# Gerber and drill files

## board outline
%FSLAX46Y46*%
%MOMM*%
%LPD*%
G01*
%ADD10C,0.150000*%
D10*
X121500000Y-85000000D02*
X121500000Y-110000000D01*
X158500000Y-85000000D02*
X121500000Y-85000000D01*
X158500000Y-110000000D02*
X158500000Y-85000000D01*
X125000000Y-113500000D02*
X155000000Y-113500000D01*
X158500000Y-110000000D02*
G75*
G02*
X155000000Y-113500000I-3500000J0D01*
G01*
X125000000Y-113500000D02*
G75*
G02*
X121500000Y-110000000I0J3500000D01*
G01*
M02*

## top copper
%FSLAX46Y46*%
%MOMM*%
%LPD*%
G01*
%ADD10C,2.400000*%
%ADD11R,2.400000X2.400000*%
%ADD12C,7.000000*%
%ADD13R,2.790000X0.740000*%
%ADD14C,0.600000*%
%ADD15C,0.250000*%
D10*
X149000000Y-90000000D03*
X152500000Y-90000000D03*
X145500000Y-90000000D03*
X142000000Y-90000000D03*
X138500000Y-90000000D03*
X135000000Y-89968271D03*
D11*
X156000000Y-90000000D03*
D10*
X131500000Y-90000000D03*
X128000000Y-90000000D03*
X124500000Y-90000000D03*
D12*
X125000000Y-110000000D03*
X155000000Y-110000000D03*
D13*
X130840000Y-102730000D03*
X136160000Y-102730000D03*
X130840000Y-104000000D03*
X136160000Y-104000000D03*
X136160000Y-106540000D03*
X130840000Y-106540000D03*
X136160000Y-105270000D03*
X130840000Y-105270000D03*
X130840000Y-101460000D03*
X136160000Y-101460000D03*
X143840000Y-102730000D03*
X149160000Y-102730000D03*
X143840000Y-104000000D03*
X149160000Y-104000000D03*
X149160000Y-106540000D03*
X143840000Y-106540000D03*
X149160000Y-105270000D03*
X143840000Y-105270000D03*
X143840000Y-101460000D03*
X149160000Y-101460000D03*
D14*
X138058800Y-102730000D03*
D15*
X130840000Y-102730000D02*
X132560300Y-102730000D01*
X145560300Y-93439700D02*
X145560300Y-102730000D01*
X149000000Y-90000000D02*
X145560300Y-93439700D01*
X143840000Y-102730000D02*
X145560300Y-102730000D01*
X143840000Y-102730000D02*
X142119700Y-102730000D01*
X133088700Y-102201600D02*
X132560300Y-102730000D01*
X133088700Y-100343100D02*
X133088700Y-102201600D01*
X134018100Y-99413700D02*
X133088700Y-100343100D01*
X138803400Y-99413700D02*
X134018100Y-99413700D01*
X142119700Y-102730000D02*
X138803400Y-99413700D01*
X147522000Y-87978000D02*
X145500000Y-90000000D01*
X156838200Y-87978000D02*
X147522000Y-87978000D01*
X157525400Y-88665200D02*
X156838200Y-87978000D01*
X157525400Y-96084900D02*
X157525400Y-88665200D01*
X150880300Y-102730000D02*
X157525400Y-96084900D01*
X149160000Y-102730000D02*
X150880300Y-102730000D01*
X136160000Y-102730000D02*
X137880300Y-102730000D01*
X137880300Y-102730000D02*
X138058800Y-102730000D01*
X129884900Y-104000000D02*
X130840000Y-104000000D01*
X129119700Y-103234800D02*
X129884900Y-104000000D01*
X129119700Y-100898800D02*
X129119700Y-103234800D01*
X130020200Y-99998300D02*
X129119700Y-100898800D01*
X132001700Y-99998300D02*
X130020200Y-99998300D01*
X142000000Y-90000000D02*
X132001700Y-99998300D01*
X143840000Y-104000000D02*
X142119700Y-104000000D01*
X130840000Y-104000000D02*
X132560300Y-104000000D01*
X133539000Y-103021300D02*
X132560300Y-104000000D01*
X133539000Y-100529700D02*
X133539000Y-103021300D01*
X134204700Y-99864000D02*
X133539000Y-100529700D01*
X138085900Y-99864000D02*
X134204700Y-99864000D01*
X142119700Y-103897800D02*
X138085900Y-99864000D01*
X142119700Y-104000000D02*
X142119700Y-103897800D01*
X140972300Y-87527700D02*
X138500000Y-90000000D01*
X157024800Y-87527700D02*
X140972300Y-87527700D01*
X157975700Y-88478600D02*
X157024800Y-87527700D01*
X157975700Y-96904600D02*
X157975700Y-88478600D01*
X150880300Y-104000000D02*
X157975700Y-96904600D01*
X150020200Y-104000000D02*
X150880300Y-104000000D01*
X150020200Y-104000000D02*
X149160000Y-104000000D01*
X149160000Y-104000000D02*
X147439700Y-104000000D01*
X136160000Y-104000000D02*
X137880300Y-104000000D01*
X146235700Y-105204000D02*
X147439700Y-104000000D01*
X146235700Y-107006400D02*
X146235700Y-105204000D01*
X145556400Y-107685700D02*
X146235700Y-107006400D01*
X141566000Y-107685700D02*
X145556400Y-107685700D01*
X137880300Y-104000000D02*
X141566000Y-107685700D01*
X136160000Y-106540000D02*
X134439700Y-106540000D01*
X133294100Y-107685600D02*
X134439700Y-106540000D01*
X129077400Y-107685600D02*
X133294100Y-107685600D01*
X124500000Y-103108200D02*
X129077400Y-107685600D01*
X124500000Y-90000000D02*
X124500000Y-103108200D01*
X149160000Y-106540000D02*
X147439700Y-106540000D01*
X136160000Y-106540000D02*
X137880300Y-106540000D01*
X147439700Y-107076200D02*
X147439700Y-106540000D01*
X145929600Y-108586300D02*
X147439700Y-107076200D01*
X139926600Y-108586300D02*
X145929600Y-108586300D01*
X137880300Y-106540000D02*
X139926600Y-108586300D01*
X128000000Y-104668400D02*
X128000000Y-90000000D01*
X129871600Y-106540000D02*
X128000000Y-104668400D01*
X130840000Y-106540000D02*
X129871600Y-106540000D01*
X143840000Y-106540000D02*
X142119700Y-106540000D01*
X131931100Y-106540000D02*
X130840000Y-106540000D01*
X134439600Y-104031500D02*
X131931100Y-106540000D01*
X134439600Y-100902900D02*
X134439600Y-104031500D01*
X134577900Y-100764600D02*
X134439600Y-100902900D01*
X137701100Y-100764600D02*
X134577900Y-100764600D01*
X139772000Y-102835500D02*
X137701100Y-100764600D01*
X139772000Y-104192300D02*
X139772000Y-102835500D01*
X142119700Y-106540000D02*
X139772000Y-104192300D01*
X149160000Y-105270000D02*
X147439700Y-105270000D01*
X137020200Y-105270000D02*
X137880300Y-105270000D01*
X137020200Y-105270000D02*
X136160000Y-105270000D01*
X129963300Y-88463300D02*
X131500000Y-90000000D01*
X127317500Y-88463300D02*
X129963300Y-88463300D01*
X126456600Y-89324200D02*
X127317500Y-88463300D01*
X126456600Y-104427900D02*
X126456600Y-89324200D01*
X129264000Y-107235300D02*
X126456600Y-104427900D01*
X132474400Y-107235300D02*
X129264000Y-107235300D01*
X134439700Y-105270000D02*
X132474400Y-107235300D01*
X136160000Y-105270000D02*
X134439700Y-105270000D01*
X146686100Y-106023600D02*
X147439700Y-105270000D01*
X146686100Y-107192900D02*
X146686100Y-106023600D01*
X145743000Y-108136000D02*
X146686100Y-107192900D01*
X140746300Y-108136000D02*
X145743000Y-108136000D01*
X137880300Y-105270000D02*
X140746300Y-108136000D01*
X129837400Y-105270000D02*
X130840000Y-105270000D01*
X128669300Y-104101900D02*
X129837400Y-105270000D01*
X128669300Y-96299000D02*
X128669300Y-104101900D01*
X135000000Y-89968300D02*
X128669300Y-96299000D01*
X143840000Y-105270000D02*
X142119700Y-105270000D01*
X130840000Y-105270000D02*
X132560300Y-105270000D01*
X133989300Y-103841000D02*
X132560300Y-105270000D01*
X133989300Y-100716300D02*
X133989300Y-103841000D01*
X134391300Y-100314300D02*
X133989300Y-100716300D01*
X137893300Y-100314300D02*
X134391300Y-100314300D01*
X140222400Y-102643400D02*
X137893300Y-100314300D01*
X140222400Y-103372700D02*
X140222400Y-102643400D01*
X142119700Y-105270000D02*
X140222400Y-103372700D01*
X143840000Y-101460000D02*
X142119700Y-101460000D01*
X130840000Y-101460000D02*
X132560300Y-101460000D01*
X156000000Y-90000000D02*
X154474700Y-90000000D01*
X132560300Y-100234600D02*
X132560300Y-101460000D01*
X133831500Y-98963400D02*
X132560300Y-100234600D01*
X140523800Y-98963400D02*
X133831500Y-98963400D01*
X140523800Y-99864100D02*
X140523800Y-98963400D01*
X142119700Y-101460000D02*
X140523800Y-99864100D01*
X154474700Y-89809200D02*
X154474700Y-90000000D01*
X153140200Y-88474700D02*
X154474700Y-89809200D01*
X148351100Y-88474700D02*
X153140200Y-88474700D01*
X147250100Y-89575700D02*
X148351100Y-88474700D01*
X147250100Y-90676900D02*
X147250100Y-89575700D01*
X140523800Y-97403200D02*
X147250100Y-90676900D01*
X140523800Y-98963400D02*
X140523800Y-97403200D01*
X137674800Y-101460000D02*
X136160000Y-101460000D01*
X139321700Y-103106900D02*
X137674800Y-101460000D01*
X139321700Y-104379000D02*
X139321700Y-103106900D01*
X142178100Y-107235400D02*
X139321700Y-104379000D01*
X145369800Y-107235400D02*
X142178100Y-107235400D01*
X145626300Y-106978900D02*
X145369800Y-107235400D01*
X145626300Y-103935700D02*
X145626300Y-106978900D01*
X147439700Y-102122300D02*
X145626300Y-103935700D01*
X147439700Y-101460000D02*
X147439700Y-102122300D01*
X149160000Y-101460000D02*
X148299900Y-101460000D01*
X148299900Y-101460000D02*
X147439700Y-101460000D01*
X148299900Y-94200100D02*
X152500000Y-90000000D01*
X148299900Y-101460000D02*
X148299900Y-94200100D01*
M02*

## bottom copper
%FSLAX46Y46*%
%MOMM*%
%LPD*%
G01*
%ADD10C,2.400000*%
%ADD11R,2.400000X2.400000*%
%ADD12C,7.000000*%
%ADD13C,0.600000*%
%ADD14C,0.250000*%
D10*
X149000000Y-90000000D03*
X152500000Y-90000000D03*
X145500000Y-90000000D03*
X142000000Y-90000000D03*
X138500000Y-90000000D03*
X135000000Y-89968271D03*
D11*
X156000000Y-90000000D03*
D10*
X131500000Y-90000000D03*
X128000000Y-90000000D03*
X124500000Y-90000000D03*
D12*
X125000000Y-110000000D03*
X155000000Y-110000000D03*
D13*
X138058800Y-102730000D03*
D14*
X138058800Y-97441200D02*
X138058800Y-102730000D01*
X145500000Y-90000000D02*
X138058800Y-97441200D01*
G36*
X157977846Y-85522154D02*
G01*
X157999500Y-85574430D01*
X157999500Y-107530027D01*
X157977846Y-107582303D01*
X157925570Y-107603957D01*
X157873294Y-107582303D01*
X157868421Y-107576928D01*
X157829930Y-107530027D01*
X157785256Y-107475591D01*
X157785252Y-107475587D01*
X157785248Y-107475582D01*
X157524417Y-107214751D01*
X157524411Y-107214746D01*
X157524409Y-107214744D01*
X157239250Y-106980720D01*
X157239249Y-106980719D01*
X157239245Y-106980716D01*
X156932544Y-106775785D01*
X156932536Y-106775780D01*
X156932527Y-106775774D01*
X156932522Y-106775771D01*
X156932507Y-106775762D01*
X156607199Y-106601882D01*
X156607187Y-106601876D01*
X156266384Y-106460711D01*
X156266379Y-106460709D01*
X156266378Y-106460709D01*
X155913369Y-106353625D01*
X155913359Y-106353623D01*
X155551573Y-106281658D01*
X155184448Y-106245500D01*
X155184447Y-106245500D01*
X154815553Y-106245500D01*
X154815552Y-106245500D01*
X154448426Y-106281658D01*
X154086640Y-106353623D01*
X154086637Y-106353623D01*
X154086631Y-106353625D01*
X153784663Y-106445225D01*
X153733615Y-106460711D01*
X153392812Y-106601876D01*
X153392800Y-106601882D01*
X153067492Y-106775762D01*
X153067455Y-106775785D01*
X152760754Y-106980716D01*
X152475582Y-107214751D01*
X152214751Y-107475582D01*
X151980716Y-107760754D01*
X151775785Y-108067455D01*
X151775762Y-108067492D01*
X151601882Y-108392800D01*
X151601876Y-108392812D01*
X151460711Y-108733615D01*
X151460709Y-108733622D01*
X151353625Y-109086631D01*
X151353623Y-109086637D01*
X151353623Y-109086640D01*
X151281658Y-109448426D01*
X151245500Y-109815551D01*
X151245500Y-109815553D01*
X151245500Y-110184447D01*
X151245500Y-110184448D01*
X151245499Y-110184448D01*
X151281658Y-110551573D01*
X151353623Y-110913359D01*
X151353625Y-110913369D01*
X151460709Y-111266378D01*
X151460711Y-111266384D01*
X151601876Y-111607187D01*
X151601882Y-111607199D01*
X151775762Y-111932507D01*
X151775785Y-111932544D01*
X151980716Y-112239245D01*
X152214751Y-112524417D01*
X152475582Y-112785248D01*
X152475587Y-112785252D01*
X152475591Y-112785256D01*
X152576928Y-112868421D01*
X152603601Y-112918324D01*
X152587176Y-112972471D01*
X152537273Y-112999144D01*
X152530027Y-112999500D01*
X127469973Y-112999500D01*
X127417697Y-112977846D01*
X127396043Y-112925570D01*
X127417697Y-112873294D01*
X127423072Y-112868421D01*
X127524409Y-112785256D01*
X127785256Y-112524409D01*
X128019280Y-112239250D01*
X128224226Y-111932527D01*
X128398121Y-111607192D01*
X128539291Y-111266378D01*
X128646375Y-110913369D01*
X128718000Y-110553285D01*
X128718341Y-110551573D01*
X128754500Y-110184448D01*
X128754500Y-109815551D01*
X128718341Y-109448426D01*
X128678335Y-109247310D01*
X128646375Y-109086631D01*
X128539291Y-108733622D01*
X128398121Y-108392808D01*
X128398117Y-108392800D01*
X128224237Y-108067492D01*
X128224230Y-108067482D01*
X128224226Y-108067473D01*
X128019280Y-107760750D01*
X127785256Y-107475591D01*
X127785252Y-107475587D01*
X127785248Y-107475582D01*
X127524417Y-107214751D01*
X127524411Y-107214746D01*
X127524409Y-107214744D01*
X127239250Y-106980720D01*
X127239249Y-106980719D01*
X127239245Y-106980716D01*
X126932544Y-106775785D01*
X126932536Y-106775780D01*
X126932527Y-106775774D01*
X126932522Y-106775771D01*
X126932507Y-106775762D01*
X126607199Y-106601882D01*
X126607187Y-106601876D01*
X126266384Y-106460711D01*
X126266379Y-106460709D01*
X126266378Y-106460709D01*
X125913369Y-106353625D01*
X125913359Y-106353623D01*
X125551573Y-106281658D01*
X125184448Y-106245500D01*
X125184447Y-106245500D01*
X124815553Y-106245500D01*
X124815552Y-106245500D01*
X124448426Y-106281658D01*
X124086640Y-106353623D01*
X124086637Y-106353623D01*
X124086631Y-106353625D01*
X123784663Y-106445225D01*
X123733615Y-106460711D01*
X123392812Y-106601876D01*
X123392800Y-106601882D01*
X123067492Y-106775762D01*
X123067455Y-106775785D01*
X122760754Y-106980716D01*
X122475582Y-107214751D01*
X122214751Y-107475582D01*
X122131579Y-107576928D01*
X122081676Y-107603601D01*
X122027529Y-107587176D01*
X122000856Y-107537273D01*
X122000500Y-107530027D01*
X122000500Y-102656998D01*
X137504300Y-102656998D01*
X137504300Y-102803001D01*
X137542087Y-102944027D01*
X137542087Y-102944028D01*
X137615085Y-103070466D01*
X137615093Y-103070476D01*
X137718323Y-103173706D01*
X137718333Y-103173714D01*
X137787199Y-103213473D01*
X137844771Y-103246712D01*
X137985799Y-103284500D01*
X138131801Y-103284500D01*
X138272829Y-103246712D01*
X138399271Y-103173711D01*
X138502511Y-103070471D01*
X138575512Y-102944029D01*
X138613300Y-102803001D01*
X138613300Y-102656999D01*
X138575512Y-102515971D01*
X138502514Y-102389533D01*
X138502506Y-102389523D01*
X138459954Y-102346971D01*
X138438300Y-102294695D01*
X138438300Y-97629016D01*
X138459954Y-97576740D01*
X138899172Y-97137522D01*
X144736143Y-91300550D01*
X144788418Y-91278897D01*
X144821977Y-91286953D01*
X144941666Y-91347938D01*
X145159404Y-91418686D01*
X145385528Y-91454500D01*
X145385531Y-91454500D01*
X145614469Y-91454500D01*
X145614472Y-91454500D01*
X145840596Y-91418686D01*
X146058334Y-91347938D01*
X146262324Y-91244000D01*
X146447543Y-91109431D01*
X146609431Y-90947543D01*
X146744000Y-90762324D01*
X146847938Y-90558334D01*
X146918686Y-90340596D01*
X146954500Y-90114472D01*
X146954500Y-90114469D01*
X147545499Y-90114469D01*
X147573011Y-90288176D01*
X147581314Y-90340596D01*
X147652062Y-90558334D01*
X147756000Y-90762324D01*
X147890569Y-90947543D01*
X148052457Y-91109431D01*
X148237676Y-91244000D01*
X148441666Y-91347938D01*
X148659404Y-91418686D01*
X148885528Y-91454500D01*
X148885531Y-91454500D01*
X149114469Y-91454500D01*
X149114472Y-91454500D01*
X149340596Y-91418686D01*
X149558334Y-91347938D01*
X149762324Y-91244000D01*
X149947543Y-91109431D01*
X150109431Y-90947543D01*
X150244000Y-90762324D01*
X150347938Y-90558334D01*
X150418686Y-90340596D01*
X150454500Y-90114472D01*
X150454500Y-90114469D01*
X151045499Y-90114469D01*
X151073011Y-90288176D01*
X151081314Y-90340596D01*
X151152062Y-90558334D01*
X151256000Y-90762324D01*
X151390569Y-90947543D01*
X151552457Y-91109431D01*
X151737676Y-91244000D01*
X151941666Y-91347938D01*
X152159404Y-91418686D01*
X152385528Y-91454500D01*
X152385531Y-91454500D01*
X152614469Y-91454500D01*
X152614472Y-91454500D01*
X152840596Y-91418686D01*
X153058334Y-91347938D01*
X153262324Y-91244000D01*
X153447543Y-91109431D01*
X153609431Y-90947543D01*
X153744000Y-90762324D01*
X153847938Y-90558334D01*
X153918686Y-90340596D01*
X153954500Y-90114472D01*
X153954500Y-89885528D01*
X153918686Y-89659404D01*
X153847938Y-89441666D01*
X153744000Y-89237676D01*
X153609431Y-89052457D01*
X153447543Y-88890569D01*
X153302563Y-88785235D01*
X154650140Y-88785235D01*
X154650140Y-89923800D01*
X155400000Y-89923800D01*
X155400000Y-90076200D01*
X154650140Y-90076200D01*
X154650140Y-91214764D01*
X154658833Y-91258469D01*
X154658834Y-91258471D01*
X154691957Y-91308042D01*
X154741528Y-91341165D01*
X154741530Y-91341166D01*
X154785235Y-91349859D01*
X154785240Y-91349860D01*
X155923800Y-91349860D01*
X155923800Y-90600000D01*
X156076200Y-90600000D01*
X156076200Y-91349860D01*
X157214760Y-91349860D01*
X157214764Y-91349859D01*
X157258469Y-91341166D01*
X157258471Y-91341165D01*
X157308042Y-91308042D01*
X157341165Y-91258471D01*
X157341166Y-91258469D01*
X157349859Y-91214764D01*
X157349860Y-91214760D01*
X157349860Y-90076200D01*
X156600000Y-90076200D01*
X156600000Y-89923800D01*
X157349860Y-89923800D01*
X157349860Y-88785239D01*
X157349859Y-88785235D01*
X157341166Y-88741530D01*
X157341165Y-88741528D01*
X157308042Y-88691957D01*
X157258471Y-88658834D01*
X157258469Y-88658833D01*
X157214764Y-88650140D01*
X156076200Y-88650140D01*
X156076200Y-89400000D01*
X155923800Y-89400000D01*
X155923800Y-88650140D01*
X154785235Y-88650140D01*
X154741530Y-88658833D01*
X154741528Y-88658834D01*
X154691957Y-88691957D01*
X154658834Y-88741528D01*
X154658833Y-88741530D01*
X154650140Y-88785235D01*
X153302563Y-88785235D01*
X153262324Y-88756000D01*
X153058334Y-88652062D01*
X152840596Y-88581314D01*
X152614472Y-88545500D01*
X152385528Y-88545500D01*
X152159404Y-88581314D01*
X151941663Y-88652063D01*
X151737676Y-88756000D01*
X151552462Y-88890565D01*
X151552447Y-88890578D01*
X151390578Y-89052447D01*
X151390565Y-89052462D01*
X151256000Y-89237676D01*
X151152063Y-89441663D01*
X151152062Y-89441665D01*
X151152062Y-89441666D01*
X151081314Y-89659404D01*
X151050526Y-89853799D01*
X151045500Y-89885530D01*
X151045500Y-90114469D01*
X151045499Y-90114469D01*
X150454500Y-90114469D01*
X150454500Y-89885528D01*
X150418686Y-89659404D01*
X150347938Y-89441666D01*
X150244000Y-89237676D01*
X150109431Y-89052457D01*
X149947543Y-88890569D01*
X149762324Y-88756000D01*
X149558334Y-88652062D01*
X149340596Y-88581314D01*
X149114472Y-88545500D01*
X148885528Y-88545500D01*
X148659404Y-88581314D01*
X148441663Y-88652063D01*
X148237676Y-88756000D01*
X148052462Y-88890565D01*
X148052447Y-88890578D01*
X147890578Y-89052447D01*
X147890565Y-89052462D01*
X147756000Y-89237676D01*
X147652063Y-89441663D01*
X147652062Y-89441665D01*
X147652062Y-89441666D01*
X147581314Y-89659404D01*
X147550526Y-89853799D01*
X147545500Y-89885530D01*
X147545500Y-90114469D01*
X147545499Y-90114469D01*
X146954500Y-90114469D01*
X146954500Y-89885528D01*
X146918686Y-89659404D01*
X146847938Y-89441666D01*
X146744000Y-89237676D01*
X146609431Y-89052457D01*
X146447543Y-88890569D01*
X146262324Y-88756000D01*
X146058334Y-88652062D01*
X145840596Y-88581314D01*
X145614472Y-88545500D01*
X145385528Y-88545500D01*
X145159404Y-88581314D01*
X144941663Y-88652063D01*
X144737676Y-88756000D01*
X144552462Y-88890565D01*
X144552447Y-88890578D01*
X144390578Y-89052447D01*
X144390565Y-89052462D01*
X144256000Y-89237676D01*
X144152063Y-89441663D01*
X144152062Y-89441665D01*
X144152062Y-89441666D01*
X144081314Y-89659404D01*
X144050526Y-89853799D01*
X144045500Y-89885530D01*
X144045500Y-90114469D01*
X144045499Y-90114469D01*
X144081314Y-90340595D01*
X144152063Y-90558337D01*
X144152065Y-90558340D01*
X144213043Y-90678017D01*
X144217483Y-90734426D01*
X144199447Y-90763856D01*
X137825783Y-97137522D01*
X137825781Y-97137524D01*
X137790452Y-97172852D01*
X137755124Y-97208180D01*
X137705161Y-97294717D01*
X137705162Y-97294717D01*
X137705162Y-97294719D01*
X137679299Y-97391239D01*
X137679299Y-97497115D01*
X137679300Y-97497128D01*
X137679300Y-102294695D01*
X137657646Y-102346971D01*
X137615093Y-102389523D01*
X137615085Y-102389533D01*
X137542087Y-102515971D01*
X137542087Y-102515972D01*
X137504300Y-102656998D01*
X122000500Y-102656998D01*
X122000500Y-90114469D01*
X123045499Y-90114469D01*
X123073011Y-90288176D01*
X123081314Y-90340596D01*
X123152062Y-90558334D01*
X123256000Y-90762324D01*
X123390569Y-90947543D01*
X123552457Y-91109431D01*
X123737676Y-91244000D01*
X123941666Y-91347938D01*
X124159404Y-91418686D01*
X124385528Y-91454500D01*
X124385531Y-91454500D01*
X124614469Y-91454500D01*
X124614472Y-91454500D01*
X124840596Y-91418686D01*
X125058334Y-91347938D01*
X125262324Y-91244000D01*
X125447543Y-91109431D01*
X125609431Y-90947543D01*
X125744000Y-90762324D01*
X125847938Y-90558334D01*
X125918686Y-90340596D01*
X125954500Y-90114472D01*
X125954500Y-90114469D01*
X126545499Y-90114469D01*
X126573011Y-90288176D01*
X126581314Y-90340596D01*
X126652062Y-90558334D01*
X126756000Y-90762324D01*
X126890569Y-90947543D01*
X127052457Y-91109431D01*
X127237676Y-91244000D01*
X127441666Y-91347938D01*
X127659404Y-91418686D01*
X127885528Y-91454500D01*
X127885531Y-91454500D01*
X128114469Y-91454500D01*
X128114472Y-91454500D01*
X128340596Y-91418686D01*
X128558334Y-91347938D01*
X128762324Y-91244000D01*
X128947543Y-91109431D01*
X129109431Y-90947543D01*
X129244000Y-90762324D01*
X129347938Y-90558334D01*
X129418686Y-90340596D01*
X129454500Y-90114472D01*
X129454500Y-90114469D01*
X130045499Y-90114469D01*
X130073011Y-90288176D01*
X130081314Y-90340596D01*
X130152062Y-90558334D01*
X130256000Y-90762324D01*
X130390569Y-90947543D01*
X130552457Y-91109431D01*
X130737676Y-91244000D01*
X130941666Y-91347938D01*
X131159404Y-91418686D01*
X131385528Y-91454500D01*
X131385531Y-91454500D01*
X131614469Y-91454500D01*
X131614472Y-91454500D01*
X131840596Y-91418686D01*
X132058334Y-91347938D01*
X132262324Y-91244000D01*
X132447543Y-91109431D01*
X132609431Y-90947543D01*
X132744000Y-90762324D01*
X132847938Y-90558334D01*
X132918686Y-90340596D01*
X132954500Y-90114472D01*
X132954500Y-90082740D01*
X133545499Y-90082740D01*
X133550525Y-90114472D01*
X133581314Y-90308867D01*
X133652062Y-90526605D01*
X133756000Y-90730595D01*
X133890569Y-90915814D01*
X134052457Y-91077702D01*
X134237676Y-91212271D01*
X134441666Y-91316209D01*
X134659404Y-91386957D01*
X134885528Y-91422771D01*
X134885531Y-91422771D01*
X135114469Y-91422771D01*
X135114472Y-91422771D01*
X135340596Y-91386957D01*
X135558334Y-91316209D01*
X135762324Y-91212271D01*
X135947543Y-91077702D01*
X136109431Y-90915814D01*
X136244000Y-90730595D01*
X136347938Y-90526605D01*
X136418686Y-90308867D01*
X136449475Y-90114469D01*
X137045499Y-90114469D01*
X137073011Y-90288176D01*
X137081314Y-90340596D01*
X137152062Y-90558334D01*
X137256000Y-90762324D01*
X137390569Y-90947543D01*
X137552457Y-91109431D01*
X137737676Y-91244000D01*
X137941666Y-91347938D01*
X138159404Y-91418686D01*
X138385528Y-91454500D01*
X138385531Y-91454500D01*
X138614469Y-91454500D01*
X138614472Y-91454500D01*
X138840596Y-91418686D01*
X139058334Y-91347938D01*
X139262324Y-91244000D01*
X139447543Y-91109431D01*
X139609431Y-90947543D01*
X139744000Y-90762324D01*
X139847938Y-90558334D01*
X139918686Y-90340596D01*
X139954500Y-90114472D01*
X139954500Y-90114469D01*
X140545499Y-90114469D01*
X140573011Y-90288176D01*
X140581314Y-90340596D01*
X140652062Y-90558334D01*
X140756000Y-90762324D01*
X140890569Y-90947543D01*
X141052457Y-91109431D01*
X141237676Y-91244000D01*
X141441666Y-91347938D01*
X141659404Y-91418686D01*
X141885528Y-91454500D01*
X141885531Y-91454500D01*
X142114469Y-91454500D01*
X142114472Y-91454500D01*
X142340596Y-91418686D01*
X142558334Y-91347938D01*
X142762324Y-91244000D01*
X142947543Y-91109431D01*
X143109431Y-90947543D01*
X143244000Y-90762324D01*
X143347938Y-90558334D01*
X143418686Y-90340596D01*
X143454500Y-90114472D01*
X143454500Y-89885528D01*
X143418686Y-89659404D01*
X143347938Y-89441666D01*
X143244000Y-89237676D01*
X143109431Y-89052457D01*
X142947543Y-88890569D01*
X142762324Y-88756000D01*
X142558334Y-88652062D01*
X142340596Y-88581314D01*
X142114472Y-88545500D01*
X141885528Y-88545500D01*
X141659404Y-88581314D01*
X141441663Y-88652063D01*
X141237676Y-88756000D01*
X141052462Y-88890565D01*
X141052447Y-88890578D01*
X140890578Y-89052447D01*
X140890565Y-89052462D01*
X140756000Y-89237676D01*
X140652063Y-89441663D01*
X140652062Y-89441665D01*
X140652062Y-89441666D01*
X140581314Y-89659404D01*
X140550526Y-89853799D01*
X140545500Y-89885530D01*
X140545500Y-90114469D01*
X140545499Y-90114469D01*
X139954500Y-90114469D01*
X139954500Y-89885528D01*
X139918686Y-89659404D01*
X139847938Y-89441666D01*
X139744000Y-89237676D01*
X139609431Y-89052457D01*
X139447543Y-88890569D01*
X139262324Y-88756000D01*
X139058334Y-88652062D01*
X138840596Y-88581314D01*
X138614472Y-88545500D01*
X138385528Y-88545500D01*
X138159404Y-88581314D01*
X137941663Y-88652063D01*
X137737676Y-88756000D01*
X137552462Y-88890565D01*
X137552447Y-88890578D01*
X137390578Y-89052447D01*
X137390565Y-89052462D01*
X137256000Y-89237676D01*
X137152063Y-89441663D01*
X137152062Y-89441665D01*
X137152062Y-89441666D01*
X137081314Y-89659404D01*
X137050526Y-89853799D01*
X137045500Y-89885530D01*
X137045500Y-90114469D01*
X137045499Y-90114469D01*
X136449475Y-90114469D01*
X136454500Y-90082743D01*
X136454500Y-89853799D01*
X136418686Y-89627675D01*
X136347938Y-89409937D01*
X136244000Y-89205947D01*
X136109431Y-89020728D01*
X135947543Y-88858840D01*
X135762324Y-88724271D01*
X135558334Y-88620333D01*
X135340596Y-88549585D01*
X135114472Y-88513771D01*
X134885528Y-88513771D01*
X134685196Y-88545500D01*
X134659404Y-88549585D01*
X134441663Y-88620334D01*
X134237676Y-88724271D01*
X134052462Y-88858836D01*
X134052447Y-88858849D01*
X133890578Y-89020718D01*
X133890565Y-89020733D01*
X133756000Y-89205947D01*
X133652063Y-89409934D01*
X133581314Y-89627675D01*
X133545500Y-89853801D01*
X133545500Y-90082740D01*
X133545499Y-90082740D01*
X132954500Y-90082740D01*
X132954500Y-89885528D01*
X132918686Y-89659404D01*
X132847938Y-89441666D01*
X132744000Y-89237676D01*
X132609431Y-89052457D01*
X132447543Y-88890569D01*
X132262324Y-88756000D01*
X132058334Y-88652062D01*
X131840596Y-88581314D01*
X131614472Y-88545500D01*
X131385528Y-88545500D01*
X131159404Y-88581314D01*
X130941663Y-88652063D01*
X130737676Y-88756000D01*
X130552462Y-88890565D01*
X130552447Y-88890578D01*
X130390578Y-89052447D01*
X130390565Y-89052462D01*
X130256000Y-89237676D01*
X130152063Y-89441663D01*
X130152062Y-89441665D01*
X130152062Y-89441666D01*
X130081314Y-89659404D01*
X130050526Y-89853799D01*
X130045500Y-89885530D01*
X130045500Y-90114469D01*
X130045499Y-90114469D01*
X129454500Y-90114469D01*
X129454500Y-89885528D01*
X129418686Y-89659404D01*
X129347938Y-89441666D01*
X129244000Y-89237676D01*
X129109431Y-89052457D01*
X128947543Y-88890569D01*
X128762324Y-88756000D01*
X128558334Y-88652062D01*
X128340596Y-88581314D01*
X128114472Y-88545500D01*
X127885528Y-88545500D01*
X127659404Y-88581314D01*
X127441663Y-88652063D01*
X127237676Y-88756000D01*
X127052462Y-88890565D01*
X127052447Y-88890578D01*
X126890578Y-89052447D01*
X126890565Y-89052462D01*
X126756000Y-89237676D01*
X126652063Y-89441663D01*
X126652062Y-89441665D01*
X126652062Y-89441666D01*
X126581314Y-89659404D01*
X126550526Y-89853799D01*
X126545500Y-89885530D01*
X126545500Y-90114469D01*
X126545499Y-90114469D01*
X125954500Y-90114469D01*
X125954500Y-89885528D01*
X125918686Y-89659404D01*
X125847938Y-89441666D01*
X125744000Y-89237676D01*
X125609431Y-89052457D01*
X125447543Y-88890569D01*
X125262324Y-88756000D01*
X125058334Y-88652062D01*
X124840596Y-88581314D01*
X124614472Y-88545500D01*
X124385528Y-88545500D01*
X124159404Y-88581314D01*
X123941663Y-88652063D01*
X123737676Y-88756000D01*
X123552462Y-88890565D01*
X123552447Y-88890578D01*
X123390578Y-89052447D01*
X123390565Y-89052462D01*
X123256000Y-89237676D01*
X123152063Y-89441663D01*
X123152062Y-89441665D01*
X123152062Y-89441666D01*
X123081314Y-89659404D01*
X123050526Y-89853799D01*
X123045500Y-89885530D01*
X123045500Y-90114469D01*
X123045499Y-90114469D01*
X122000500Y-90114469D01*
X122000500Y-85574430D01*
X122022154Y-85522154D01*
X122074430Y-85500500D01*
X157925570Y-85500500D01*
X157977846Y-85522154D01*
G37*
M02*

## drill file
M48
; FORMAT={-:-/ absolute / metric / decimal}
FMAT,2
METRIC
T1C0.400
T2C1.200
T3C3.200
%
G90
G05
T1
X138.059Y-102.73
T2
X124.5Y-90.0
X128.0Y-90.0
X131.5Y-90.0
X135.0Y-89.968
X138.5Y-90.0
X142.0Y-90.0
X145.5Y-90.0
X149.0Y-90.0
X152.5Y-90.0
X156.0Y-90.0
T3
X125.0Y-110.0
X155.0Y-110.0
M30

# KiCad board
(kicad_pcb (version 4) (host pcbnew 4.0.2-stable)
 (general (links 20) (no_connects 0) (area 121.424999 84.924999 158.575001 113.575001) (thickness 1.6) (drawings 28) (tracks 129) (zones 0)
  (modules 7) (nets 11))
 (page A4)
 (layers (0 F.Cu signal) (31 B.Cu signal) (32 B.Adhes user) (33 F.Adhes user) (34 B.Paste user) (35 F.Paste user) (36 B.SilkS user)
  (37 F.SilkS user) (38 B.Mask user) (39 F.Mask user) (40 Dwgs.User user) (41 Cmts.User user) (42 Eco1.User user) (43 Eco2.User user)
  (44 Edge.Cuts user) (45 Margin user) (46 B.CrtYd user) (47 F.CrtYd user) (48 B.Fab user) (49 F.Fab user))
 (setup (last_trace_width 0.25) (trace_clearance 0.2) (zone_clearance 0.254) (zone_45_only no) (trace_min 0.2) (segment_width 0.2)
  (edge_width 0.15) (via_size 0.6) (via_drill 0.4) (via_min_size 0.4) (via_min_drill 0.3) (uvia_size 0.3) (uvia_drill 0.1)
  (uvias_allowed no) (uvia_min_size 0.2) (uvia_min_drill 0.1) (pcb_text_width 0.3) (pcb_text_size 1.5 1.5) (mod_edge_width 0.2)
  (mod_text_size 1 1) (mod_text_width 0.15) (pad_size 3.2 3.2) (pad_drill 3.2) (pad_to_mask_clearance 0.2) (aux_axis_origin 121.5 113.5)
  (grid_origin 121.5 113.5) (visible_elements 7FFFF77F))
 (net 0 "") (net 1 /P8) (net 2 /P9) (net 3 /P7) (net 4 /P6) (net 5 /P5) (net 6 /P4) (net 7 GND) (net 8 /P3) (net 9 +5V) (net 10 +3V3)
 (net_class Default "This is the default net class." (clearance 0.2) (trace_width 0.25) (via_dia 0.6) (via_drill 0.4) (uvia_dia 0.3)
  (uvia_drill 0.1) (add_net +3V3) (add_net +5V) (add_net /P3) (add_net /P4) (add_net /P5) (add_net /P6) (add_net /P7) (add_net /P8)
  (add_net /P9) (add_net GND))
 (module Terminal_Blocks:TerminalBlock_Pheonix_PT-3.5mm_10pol (layer F.Cu) (at 156 90 180)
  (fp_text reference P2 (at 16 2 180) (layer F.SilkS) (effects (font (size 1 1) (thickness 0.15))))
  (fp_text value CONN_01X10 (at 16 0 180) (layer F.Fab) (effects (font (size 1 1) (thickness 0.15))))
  (pad 3 thru_hole circle (at 7 0) (size 2.4 2.4) (drill 1.2) (layers *.Cu *.Mask F.SilkS) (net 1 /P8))
  (pad 2 thru_hole circle (at 3.5 0) (size 2.4 2.4) (drill 1.2) (layers *.Cu *.Mask F.SilkS) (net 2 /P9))
  (pad 4 thru_hole circle (at 10.5 0) (size 2.4 2.4) (drill 1.2) (layers *.Cu *.Mask F.SilkS) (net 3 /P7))
  (pad 5 thru_hole circle (at 14 0) (size 2.4 2.4) (drill 1.2) (layers *.Cu *.Mask F.SilkS) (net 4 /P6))
  (pad 6 thru_hole circle (at 17.5 0) (size 2.4 2.4) (drill 1.2) (layers *.Cu *.Mask F.SilkS) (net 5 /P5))
  (pad 7 thru_hole circle (at 21 0.031729) (size 2.4 2.4) (drill 1.2) (layers *.Cu *.Mask F.SilkS) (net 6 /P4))
  (pad 1 thru_hole rect (at 0 0) (size 2.4 2.4) (drill 1.2) (layers *.Cu *.Mask F.SilkS) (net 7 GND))
  (pad 8 thru_hole circle (at 24.5 0) (size 2.4 2.4) (drill 1.2) (layers *.Cu *.Mask F.SilkS) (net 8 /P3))
  (pad 9 thru_hole circle (at 28 0) (size 2.4 2.4) (drill 1.2) (layers *.Cu *.Mask F.SilkS) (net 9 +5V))
  (pad 10 thru_hole circle (at 31.5 0) (size 2.4 2.4) (drill 1.2) (layers *.Cu *.Mask F.SilkS) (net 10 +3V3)))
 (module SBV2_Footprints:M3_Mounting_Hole (layer F.Cu) (at 125 110)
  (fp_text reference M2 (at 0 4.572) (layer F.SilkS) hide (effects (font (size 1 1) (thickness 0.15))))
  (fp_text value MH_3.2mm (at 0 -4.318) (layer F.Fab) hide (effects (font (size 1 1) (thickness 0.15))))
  (pad "" np_thru_hole circle (at 0 0) (size 7 7) (drill 3.2) (layers *.Cu *.Mask)))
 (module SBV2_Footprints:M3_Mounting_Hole (layer F.Cu) (at 155 110)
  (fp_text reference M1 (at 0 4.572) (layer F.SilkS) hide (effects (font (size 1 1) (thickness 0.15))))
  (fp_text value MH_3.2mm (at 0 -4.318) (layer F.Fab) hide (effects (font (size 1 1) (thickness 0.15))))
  (pad "" np_thru_hole circle (at 0 0) (size 7 7) (drill 3.2) (layers *.Cu *.Mask)))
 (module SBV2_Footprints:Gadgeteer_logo (layer F.Cu) (at 125 103.5)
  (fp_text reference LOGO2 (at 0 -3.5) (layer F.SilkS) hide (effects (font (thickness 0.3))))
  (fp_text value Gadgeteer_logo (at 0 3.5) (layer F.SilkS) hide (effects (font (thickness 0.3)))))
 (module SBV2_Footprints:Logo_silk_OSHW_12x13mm (layer B.Cu) (at 139.5 99.5 180)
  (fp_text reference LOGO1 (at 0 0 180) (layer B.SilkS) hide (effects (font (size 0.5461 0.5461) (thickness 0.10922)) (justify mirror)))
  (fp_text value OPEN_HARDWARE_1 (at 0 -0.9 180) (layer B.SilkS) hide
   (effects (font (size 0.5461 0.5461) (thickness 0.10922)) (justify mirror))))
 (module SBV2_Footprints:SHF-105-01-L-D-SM (layer F.Cu) (at 133.5 104 90)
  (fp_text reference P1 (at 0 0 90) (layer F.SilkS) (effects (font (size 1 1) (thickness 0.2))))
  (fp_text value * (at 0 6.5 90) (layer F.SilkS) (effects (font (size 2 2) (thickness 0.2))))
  (pad 8 smd rect (at 1.27 -2.66 90) (size 0.74 2.79) (layers F.Cu F.Paste F.Mask) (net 1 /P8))
  (pad 7 smd rect (at 1.27 2.66 90) (size 0.74 2.79) (layers F.Cu F.Paste F.Mask) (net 3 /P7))
  (pad 6 smd rect (at 0 -2.66 90) (size 0.74 2.79) (layers F.Cu F.Paste F.Mask) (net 4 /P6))
  (pad 5 smd rect (at 0 2.66 270) (size 0.74 2.79) (layers F.Cu F.Paste F.Mask) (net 5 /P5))
  (pad 1 smd rect (at -2.54 2.66 90) (size 0.74 2.79) (layers F.Cu F.Paste F.Mask) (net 10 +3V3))
  (pad 2 smd rect (at -2.54 -2.66 90) (size 0.74 2.79) (layers F.Cu F.Paste F.Mask) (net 9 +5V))
  (pad 3 smd rect (at -1.27 2.66 90) (size 0.74 2.79) (layers F.Cu F.Paste F.Mask) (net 8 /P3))
  (pad 4 smd rect (at -1.27 -2.66 90) (size 0.74 2.79) (layers F.Cu F.Paste F.Mask) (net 6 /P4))
  (pad 10 smd rect (at 2.54 -2.66 90) (size 0.74 2.79) (layers F.Cu F.Paste F.Mask) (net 7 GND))
  (pad 9 smd rect (at 2.54 2.66 90) (size 0.74 2.79) (layers F.Cu F.Paste F.Mask) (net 2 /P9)))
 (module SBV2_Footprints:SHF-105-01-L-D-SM (layer F.Cu) (at 146.5 104 90)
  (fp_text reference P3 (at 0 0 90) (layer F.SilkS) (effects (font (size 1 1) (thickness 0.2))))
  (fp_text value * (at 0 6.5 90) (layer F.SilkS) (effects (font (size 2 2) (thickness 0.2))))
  (pad 8 smd rect (at 1.27 -2.66 90) (size 0.74 2.79) (layers F.Cu F.Paste F.Mask) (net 1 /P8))
  (pad 7 smd rect (at 1.27 2.66 90) (size 0.74 2.79) (layers F.Cu F.Paste F.Mask) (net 3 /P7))
  (pad 6 smd rect (at 0 -2.66 90) (size 0.74 2.79) (layers F.Cu F.Paste F.Mask) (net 4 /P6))
  (pad 5 smd rect (at 0 2.66 270) (size 0.74 2.79) (layers F.Cu F.Paste F.Mask) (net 5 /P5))
  (pad 1 smd rect (at -2.54 2.66 90) (size 0.74 2.79) (layers F.Cu F.Paste F.Mask) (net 10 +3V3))
  (pad 2 smd rect (at -2.54 -2.66 90) (size 0.74 2.79) (layers F.Cu F.Paste F.Mask) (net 9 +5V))
  (pad 3 smd rect (at -1.27 2.66 90) (size 0.74 2.79) (layers F.Cu F.Paste F.Mask) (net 8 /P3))
  (pad 4 smd rect (at -1.27 -2.66 90) (size 0.74 2.79) (layers F.Cu F.Paste F.Mask) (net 6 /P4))
  (pad 10 smd rect (at 2.54 -2.66 90) (size 0.74 2.79) (layers F.Cu F.Paste F.Mask) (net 7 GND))
  (pad 9 smd rect (at 2.54 2.66 90) (size 0.74 2.79) (layers F.Cu F.Paste F.Mask) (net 2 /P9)))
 (gr_line (start 121.5 85) (end 121.5 110) (angle 90) (layer Edge.Cuts) (width 0.15))
 (gr_line (start 158.5 85) (end 121.5 85) (angle 90) (layer Edge.Cuts) (width 0.15))
 (gr_line (start 158.5 110) (end 158.5 85) (angle 90) (layer Edge.Cuts) (width 0.15))
 (gr_line (start 125 113.5) (end 155 113.5) (angle 90) (layer Edge.Cuts) (width 0.15))
 (gr_arc (start 155 110) (end 158.5 110) (angle 90) (layer Edge.Cuts) (width 0.15))
 (gr_arc (start 125 110) (end 125 113.5) (angle 90) (layer Edge.Cuts) (width 0.15))
 (segment (start 130.84 102.73) (end 132.5603 102.73) (width 0.25) (layer F.Cu) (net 1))
 (segment (start 145.5603 93.4397) (end 145.5603 102.73) (width 0.25) (layer F.Cu) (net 1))
 (segment (start 149 90) (end 145.5603 93.4397) (width 0.25) (layer F.Cu) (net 1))
 (segment (start 143.84 102.73) (end 145.5603 102.73) (width 0.25) (layer F.Cu) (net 1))
 (segment (start 143.84 102.73) (end 142.1197 102.73) (width 0.25) (layer F.Cu) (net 1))
 (segment (start 133.0887 102.2016) (end 132.5603 102.73) (width 0.25) (layer F.Cu) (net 1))
 (segment (start 133.0887 100.3431) (end 133.0887 102.2016) (width 0.25) (layer F.Cu) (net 1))
 (segment (start 134.0181 99.4137) (end 133.0887 100.3431) (width 0.25) (layer F.Cu) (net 1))
 (segment (start 138.8034 99.4137) (end 134.0181 99.4137) (width 0.25) (layer F.Cu) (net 1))
 (segment (start 142.1197 102.73) (end 138.8034 99.4137) (width 0.25) (layer F.Cu) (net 1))
 (via (at 138.0588 102.73) (size 0.6) (layers F.Cu B.Cu) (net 3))
 (segment (start 147.522 87.978) (end 145.5 90) (width 0.25) (layer F.Cu) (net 3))
 (segment (start 156.8382 87.978) (end 147.522 87.978) (width 0.25) (layer F.Cu) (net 3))
 (segment (start 157.5254 88.6652) (end 156.8382 87.978) (width 0.25) (layer F.Cu) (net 3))
 (segment (start 157.5254 96.0849) (end 157.5254 88.6652) (width 0.25) (layer F.Cu) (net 3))
 (segment (start 150.8803 102.73) (end 157.5254 96.0849) (width 0.25) (layer F.Cu) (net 3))
 (segment (start 149.16 102.73) (end 150.8803 102.73) (width 0.25) (layer F.Cu) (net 3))
 (segment (start 136.16 102.73) (end 137.8803 102.73) (width 0.25) (layer F.Cu) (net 3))
 (segment (start 138.0588 97.4412) (end 138.0588 102.73) (width 0.25) (layer B.Cu) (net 3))
 (segment (start 145.5 90) (end 138.0588 97.4412) (width 0.25) (layer B.Cu) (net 3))
 (segment (start 137.8803 102.73) (end 138.0588 102.73) (width 0.25) (layer F.Cu) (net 3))
 (segment (start 129.8849 104) (end 130.84 104) (width 0.25) (layer F.Cu) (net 4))
 (segment (start 129.1197 103.2348) (end 129.8849 104) (width 0.25) (layer F.Cu) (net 4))
 (segment (start 129.1197 100.8988) (end 129.1197 103.2348) (width 0.25) (layer F.Cu) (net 4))
 (segment (start 130.0202 99.9983) (end 129.1197 100.8988) (width 0.25) (layer F.Cu) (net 4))
 (segment (start 132.0017 99.9983) (end 130.0202 99.9983) (width 0.25) (layer F.Cu) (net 4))
 (segment (start 142 90) (end 132.0017 99.9983) (width 0.25) (layer F.Cu) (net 4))
 (segment (start 143.84 104) (end 142.1197 104) (width 0.25) (layer F.Cu) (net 4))
 (segment (start 130.84 104) (end 132.5603 104) (width 0.25) (layer F.Cu) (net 4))
 (segment (start 133.539 103.0213) (end 132.5603 104) (width 0.25) (layer F.Cu) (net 4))
 (segment (start 133.539 100.5297) (end 133.539 103.0213) (width 0.25) (layer F.Cu) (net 4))
 (segment (start 134.2047 99.864) (end 133.539 100.5297) (width 0.25) (layer F.Cu) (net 4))
 (segment (start 138.0859 99.864) (end 134.2047 99.864) (width 0.25) (layer F.Cu) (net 4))
 (segment (start 142.1197 103.8978) (end 138.0859 99.864) (width 0.25) (layer F.Cu) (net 4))
 (segment (start 142.1197 104) (end 142.1197 103.8978) (width 0.25) (layer F.Cu) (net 4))
 (segment (start 140.9723 87.5277) (end 138.5 90) (width 0.25) (layer F.Cu) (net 5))
 (segment (start 157.0248 87.5277) (end 140.9723 87.5277) (width 0.25) (layer F.Cu) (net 5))
 (segment (start 157.9757 88.4786) (end 157.0248 87.5277) (width 0.25) (layer F.Cu) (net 5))
 (segment (start 157.9757 96.9046) (end 157.9757 88.4786) (width 0.25) (layer F.Cu) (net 5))
 (segment (start 150.8803 104) (end 157.9757 96.9046) (width 0.25) (layer F.Cu) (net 5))
 (segment (start 150.0202 104) (end 150.8803 104) (width 0.25) (layer F.Cu) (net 5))
 (segment (start 150.0202 104) (end 149.16 104) (width 0.25) (layer F.Cu) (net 5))
 (segment (start 149.16 104) (end 147.4397 104) (width 0.25) (layer F.Cu) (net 5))
 (segment (start 136.16 104) (end 137.8803 104) (width 0.25) (layer F.Cu) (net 5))
 (segment (start 146.2357 105.204) (end 147.4397 104) (width 0.25) (layer F.Cu) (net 5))
 (segment (start 146.2357 107.0064) (end 146.2357 105.204) (width 0.25) (layer F.Cu) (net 5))
 (segment (start 145.5564 107.6857) (end 146.2357 107.0064) (width 0.25) (layer F.Cu) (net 5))
 (segment (start 141.566 107.6857) (end 145.5564 107.6857) (width 0.25) (layer F.Cu) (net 5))
 (segment (start 137.8803 104) (end 141.566 107.6857) (width 0.25) (layer F.Cu) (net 5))
 (segment (start 136.16 106.54) (end 134.4397 106.54) (width 0.25) (layer F.Cu) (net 10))
 (segment (start 133.2941 107.6856) (end 134.4397 106.54) (width 0.25) (layer F.Cu) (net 10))
 (segment (start 129.0774 107.6856) (end 133.2941 107.6856) (width 0.25) (layer F.Cu) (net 10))
 (segment (start 124.5 103.1082) (end 129.0774 107.6856) (width 0.25) (layer F.Cu) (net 10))
 (segment (start 124.5 90) (end 124.5 103.1082) (width 0.25) (layer F.Cu) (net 10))
 (segment (start 149.16 106.54) (end 147.4397 106.54) (width 0.25) (layer F.Cu) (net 10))
 (segment (start 136.16 106.54) (end 137.8803 106.54) (width 0.25) (layer F.Cu) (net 10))
 (segment (start 147.4397 107.0762) (end 147.4397 106.54) (width 0.25) (layer F.Cu) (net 10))
 (segment (start 145.9296 108.5863) (end 147.4397 107.0762) (width 0.25) (layer F.Cu) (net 10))
 (segment (start 139.9266 108.5863) (end 145.9296 108.5863) (width 0.25) (layer F.Cu) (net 10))
 (segment (start 137.8803 106.54) (end 139.9266 108.5863) (width 0.25) (layer F.Cu) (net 10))
 (segment (start 128 104.6684) (end 128 90) (width 0.25) (layer F.Cu) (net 9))
 (segment (start 129.8716 106.54) (end 128 104.6684) (width 0.25) (layer F.Cu) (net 9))
 (segment (start 130.84 106.54) (end 129.8716 106.54) (width 0.25) (layer F.Cu) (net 9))
 (segment (start 143.84 106.54) (end 142.1197 106.54) (width 0.25) (layer F.Cu) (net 9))
 (segment (start 131.9311 106.54) (end 130.84 106.54) (width 0.25) (layer F.Cu) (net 9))
 (segment (start 134.4396 104.0315) (end 131.9311 106.54) (width 0.25) (layer F.Cu) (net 9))
 (segment (start 134.4396 100.9029) (end 134.4396 104.0315) (width 0.25) (layer F.Cu) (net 9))
 (segment (start 134.5779 100.7646) (end 134.4396 100.9029) (width 0.25) (layer F.Cu) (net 9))
 (segment (start 137.7011 100.7646) (end 134.5779 100.7646) (width 0.25) (layer F.Cu) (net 9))
 (segment (start 139.772 102.8355) (end 137.7011 100.7646) (width 0.25) (layer F.Cu) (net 9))
 (segment (start 139.772 104.1923) (end 139.772 102.8355) (width 0.25) (layer F.Cu) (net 9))
 (segment (start 142.1197 106.54) (end 139.772 104.1923) (width 0.25) (layer F.Cu) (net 9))
 (segment (start 149.16 105.27) (end 147.4397 105.27) (width 0.25) (layer F.Cu) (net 8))
 (segment (start 137.0202 105.27) (end 137.8803 105.27) (width 0.25) (layer F.Cu) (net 8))
 (segment (start 137.0202 105.27) (end 136.16 105.27) (width 0.25) (layer F.Cu) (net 8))
 (segment (start 129.9633 88.4633) (end 131.5 90) (width 0.25) (layer F.Cu) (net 8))
 (segment (start 127.3175 88.4633) (end 129.9633 88.4633) (width 0.25) (layer F.Cu) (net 8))
 (segment (start 126.4566 89.3242) (end 127.3175 88.4633) (width 0.25) (layer F.Cu) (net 8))
 (segment (start 126.4566 104.4279) (end 126.4566 89.3242) (width 0.25) (layer F.Cu) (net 8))
 (segment (start 129.264 107.2353) (end 126.4566 104.4279) (width 0.25) (layer F.Cu) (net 8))
 (segment (start 132.4744 107.2353) (end 129.264 107.2353) (width 0.25) (layer F.Cu) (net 8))
 (segment (start 134.4397 105.27) (end 132.4744 107.2353) (width 0.25) (layer F.Cu) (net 8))
 (segment (start 136.16 105.27) (end 134.4397 105.27) (width 0.25) (layer F.Cu) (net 8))
 (segment (start 146.6861 106.0236) (end 147.4397 105.27) (width 0.25) (layer F.Cu) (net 8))
 (segment (start 146.6861 107.1929) (end 146.6861 106.0236) (width 0.25) (layer F.Cu) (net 8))
 (segment (start 145.743 108.136) (end 146.6861 107.1929) (width 0.25) (layer F.Cu) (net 8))
 (segment (start 140.7463 108.136) (end 145.743 108.136) (width 0.25) (layer F.Cu) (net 8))
 (segment (start 137.8803 105.27) (end 140.7463 108.136) (width 0.25) (layer F.Cu) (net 8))
 (segment (start 129.8374 105.27) (end 130.84 105.27) (width 0.25) (layer F.Cu) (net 6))
 (segment (start 128.6693 104.1019) (end 129.8374 105.27) (width 0.25) (layer F.Cu) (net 6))
 (segment (start 128.6693 96.299) (end 128.6693 104.1019) (width 0.25) (layer F.Cu) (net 6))
 (segment (start 135 89.9683) (end 128.6693 96.299) (width 0.25) (layer F.Cu) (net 6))
 (segment (start 143.84 105.27) (end 142.1197 105.27) (width 0.25) (layer F.Cu) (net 6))
 (segment (start 130.84 105.27) (end 132.5603 105.27) (width 0.25) (layer F.Cu) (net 6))
 (segment (start 133.9893 103.841) (end 132.5603 105.27) (width 0.25) (layer F.Cu) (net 6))
 (segment (start 133.9893 100.7163) (end 133.9893 103.841) (width 0.25) (layer F.Cu) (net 6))
 (segment (start 134.3913 100.3143) (end 133.9893 100.7163) (width 0.25) (layer F.Cu) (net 6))
 (segment (start 137.8933 100.3143) (end 134.3913 100.3143) (width 0.25) (layer F.Cu) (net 6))
 (segment (start 140.2224 102.6434) (end 137.8933 100.3143) (width 0.25) (layer F.Cu) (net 6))
 (segment (start 140.2224 103.3727) (end 140.2224 102.6434) (width 0.25) (layer F.Cu) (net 6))
 (segment (start 142.1197 105.27) (end 140.2224 103.3727) (width 0.25) (layer F.Cu) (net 6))
 (segment (start 143.84 101.46) (end 142.1197 101.46) (width 0.25) (layer F.Cu) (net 7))
 (segment (start 130.84 101.46) (end 132.5603 101.46) (width 0.25) (layer F.Cu) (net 7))
 (segment (start 156 90) (end 154.4747 90) (width 0.25) (layer F.Cu) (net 7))
 (segment (start 132.5603 100.2346) (end 132.5603 101.46) (width 0.25) (layer F.Cu) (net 7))
 (segment (start 133.8315 98.9634) (end 132.5603 100.2346) (width 0.25) (layer F.Cu) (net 7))
 (segment (start 140.5238 98.9634) (end 133.8315 98.9634) (width 0.25) (layer F.Cu) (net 7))
 (segment (start 140.5238 99.8641) (end 140.5238 98.9634) (width 0.25) (layer F.Cu) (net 7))
 (segment (start 142.1197 101.46) (end 140.5238 99.8641) (width 0.25) (layer F.Cu) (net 7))
 (segment (start 154.4747 89.8092) (end 154.4747 90) (width 0.25) (layer F.Cu) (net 7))
 (segment (start 153.1402 88.4747) (end 154.4747 89.8092) (width 0.25) (layer F.Cu) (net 7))
 (segment (start 148.3511 88.4747) (end 153.1402 88.4747) (width 0.25) (layer F.Cu) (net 7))
 (segment (start 147.2501 89.5757) (end 148.3511 88.4747) (width 0.25) (layer F.Cu) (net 7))
 (segment (start 147.2501 90.6769) (end 147.2501 89.5757) (width 0.25) (layer F.Cu) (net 7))
 (segment (start 140.5238 97.4032) (end 147.2501 90.6769) (width 0.25) (layer F.Cu) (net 7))
 (segment (start 140.5238 98.9634) (end 140.5238 97.4032) (width 0.25) (layer F.Cu) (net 7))
 (segment (start 137.6748 101.46) (end 136.16 101.46) (width 0.25) (layer F.Cu) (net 2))
 (segment (start 139.3217 103.1069) (end 137.6748 101.46) (width 0.25) (layer F.Cu) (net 2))
 (segment (start 139.3217 104.379) (end 139.3217 103.1069) (width 0.25) (layer F.Cu) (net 2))
 (segment (start 142.1781 107.2354) (end 139.3217 104.379) (width 0.25) (layer F.Cu) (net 2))
 (segment (start 145.3698 107.2354) (end 142.1781 107.2354) (width 0.25) (layer F.Cu) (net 2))
 (segment (start 145.6263 106.9789) (end 145.3698 107.2354) (width 0.25) (layer F.Cu) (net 2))
 (segment (start 145.6263 103.9357) (end 145.6263 106.9789) (width 0.25) (layer F.Cu) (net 2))
 (segment (start 147.4397 102.1223) (end 145.6263 103.9357) (width 0.25) (layer F.Cu) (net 2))
 (segment (start 147.4397 101.46) (end 147.4397 102.1223) (width 0.25) (layer F.Cu) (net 2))
 (segment (start 149.16 101.46) (end 148.2999 101.46) (width 0.25) (layer F.Cu) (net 2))
 (segment (start 148.2999 101.46) (end 147.4397 101.46) (width 0.25) (layer F.Cu) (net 2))
 (segment (start 148.2999 94.2001) (end 152.5 90) (width 0.25) (layer F.Cu) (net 2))
 (segment (start 148.2999 101.46) (end 148.2999 94.2001) (width 0.25) (layer F.Cu) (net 2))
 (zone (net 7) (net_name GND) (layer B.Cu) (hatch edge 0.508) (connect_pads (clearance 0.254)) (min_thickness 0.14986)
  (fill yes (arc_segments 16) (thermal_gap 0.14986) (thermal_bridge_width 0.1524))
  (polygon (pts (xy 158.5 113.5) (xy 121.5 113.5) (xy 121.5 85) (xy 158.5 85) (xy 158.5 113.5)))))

